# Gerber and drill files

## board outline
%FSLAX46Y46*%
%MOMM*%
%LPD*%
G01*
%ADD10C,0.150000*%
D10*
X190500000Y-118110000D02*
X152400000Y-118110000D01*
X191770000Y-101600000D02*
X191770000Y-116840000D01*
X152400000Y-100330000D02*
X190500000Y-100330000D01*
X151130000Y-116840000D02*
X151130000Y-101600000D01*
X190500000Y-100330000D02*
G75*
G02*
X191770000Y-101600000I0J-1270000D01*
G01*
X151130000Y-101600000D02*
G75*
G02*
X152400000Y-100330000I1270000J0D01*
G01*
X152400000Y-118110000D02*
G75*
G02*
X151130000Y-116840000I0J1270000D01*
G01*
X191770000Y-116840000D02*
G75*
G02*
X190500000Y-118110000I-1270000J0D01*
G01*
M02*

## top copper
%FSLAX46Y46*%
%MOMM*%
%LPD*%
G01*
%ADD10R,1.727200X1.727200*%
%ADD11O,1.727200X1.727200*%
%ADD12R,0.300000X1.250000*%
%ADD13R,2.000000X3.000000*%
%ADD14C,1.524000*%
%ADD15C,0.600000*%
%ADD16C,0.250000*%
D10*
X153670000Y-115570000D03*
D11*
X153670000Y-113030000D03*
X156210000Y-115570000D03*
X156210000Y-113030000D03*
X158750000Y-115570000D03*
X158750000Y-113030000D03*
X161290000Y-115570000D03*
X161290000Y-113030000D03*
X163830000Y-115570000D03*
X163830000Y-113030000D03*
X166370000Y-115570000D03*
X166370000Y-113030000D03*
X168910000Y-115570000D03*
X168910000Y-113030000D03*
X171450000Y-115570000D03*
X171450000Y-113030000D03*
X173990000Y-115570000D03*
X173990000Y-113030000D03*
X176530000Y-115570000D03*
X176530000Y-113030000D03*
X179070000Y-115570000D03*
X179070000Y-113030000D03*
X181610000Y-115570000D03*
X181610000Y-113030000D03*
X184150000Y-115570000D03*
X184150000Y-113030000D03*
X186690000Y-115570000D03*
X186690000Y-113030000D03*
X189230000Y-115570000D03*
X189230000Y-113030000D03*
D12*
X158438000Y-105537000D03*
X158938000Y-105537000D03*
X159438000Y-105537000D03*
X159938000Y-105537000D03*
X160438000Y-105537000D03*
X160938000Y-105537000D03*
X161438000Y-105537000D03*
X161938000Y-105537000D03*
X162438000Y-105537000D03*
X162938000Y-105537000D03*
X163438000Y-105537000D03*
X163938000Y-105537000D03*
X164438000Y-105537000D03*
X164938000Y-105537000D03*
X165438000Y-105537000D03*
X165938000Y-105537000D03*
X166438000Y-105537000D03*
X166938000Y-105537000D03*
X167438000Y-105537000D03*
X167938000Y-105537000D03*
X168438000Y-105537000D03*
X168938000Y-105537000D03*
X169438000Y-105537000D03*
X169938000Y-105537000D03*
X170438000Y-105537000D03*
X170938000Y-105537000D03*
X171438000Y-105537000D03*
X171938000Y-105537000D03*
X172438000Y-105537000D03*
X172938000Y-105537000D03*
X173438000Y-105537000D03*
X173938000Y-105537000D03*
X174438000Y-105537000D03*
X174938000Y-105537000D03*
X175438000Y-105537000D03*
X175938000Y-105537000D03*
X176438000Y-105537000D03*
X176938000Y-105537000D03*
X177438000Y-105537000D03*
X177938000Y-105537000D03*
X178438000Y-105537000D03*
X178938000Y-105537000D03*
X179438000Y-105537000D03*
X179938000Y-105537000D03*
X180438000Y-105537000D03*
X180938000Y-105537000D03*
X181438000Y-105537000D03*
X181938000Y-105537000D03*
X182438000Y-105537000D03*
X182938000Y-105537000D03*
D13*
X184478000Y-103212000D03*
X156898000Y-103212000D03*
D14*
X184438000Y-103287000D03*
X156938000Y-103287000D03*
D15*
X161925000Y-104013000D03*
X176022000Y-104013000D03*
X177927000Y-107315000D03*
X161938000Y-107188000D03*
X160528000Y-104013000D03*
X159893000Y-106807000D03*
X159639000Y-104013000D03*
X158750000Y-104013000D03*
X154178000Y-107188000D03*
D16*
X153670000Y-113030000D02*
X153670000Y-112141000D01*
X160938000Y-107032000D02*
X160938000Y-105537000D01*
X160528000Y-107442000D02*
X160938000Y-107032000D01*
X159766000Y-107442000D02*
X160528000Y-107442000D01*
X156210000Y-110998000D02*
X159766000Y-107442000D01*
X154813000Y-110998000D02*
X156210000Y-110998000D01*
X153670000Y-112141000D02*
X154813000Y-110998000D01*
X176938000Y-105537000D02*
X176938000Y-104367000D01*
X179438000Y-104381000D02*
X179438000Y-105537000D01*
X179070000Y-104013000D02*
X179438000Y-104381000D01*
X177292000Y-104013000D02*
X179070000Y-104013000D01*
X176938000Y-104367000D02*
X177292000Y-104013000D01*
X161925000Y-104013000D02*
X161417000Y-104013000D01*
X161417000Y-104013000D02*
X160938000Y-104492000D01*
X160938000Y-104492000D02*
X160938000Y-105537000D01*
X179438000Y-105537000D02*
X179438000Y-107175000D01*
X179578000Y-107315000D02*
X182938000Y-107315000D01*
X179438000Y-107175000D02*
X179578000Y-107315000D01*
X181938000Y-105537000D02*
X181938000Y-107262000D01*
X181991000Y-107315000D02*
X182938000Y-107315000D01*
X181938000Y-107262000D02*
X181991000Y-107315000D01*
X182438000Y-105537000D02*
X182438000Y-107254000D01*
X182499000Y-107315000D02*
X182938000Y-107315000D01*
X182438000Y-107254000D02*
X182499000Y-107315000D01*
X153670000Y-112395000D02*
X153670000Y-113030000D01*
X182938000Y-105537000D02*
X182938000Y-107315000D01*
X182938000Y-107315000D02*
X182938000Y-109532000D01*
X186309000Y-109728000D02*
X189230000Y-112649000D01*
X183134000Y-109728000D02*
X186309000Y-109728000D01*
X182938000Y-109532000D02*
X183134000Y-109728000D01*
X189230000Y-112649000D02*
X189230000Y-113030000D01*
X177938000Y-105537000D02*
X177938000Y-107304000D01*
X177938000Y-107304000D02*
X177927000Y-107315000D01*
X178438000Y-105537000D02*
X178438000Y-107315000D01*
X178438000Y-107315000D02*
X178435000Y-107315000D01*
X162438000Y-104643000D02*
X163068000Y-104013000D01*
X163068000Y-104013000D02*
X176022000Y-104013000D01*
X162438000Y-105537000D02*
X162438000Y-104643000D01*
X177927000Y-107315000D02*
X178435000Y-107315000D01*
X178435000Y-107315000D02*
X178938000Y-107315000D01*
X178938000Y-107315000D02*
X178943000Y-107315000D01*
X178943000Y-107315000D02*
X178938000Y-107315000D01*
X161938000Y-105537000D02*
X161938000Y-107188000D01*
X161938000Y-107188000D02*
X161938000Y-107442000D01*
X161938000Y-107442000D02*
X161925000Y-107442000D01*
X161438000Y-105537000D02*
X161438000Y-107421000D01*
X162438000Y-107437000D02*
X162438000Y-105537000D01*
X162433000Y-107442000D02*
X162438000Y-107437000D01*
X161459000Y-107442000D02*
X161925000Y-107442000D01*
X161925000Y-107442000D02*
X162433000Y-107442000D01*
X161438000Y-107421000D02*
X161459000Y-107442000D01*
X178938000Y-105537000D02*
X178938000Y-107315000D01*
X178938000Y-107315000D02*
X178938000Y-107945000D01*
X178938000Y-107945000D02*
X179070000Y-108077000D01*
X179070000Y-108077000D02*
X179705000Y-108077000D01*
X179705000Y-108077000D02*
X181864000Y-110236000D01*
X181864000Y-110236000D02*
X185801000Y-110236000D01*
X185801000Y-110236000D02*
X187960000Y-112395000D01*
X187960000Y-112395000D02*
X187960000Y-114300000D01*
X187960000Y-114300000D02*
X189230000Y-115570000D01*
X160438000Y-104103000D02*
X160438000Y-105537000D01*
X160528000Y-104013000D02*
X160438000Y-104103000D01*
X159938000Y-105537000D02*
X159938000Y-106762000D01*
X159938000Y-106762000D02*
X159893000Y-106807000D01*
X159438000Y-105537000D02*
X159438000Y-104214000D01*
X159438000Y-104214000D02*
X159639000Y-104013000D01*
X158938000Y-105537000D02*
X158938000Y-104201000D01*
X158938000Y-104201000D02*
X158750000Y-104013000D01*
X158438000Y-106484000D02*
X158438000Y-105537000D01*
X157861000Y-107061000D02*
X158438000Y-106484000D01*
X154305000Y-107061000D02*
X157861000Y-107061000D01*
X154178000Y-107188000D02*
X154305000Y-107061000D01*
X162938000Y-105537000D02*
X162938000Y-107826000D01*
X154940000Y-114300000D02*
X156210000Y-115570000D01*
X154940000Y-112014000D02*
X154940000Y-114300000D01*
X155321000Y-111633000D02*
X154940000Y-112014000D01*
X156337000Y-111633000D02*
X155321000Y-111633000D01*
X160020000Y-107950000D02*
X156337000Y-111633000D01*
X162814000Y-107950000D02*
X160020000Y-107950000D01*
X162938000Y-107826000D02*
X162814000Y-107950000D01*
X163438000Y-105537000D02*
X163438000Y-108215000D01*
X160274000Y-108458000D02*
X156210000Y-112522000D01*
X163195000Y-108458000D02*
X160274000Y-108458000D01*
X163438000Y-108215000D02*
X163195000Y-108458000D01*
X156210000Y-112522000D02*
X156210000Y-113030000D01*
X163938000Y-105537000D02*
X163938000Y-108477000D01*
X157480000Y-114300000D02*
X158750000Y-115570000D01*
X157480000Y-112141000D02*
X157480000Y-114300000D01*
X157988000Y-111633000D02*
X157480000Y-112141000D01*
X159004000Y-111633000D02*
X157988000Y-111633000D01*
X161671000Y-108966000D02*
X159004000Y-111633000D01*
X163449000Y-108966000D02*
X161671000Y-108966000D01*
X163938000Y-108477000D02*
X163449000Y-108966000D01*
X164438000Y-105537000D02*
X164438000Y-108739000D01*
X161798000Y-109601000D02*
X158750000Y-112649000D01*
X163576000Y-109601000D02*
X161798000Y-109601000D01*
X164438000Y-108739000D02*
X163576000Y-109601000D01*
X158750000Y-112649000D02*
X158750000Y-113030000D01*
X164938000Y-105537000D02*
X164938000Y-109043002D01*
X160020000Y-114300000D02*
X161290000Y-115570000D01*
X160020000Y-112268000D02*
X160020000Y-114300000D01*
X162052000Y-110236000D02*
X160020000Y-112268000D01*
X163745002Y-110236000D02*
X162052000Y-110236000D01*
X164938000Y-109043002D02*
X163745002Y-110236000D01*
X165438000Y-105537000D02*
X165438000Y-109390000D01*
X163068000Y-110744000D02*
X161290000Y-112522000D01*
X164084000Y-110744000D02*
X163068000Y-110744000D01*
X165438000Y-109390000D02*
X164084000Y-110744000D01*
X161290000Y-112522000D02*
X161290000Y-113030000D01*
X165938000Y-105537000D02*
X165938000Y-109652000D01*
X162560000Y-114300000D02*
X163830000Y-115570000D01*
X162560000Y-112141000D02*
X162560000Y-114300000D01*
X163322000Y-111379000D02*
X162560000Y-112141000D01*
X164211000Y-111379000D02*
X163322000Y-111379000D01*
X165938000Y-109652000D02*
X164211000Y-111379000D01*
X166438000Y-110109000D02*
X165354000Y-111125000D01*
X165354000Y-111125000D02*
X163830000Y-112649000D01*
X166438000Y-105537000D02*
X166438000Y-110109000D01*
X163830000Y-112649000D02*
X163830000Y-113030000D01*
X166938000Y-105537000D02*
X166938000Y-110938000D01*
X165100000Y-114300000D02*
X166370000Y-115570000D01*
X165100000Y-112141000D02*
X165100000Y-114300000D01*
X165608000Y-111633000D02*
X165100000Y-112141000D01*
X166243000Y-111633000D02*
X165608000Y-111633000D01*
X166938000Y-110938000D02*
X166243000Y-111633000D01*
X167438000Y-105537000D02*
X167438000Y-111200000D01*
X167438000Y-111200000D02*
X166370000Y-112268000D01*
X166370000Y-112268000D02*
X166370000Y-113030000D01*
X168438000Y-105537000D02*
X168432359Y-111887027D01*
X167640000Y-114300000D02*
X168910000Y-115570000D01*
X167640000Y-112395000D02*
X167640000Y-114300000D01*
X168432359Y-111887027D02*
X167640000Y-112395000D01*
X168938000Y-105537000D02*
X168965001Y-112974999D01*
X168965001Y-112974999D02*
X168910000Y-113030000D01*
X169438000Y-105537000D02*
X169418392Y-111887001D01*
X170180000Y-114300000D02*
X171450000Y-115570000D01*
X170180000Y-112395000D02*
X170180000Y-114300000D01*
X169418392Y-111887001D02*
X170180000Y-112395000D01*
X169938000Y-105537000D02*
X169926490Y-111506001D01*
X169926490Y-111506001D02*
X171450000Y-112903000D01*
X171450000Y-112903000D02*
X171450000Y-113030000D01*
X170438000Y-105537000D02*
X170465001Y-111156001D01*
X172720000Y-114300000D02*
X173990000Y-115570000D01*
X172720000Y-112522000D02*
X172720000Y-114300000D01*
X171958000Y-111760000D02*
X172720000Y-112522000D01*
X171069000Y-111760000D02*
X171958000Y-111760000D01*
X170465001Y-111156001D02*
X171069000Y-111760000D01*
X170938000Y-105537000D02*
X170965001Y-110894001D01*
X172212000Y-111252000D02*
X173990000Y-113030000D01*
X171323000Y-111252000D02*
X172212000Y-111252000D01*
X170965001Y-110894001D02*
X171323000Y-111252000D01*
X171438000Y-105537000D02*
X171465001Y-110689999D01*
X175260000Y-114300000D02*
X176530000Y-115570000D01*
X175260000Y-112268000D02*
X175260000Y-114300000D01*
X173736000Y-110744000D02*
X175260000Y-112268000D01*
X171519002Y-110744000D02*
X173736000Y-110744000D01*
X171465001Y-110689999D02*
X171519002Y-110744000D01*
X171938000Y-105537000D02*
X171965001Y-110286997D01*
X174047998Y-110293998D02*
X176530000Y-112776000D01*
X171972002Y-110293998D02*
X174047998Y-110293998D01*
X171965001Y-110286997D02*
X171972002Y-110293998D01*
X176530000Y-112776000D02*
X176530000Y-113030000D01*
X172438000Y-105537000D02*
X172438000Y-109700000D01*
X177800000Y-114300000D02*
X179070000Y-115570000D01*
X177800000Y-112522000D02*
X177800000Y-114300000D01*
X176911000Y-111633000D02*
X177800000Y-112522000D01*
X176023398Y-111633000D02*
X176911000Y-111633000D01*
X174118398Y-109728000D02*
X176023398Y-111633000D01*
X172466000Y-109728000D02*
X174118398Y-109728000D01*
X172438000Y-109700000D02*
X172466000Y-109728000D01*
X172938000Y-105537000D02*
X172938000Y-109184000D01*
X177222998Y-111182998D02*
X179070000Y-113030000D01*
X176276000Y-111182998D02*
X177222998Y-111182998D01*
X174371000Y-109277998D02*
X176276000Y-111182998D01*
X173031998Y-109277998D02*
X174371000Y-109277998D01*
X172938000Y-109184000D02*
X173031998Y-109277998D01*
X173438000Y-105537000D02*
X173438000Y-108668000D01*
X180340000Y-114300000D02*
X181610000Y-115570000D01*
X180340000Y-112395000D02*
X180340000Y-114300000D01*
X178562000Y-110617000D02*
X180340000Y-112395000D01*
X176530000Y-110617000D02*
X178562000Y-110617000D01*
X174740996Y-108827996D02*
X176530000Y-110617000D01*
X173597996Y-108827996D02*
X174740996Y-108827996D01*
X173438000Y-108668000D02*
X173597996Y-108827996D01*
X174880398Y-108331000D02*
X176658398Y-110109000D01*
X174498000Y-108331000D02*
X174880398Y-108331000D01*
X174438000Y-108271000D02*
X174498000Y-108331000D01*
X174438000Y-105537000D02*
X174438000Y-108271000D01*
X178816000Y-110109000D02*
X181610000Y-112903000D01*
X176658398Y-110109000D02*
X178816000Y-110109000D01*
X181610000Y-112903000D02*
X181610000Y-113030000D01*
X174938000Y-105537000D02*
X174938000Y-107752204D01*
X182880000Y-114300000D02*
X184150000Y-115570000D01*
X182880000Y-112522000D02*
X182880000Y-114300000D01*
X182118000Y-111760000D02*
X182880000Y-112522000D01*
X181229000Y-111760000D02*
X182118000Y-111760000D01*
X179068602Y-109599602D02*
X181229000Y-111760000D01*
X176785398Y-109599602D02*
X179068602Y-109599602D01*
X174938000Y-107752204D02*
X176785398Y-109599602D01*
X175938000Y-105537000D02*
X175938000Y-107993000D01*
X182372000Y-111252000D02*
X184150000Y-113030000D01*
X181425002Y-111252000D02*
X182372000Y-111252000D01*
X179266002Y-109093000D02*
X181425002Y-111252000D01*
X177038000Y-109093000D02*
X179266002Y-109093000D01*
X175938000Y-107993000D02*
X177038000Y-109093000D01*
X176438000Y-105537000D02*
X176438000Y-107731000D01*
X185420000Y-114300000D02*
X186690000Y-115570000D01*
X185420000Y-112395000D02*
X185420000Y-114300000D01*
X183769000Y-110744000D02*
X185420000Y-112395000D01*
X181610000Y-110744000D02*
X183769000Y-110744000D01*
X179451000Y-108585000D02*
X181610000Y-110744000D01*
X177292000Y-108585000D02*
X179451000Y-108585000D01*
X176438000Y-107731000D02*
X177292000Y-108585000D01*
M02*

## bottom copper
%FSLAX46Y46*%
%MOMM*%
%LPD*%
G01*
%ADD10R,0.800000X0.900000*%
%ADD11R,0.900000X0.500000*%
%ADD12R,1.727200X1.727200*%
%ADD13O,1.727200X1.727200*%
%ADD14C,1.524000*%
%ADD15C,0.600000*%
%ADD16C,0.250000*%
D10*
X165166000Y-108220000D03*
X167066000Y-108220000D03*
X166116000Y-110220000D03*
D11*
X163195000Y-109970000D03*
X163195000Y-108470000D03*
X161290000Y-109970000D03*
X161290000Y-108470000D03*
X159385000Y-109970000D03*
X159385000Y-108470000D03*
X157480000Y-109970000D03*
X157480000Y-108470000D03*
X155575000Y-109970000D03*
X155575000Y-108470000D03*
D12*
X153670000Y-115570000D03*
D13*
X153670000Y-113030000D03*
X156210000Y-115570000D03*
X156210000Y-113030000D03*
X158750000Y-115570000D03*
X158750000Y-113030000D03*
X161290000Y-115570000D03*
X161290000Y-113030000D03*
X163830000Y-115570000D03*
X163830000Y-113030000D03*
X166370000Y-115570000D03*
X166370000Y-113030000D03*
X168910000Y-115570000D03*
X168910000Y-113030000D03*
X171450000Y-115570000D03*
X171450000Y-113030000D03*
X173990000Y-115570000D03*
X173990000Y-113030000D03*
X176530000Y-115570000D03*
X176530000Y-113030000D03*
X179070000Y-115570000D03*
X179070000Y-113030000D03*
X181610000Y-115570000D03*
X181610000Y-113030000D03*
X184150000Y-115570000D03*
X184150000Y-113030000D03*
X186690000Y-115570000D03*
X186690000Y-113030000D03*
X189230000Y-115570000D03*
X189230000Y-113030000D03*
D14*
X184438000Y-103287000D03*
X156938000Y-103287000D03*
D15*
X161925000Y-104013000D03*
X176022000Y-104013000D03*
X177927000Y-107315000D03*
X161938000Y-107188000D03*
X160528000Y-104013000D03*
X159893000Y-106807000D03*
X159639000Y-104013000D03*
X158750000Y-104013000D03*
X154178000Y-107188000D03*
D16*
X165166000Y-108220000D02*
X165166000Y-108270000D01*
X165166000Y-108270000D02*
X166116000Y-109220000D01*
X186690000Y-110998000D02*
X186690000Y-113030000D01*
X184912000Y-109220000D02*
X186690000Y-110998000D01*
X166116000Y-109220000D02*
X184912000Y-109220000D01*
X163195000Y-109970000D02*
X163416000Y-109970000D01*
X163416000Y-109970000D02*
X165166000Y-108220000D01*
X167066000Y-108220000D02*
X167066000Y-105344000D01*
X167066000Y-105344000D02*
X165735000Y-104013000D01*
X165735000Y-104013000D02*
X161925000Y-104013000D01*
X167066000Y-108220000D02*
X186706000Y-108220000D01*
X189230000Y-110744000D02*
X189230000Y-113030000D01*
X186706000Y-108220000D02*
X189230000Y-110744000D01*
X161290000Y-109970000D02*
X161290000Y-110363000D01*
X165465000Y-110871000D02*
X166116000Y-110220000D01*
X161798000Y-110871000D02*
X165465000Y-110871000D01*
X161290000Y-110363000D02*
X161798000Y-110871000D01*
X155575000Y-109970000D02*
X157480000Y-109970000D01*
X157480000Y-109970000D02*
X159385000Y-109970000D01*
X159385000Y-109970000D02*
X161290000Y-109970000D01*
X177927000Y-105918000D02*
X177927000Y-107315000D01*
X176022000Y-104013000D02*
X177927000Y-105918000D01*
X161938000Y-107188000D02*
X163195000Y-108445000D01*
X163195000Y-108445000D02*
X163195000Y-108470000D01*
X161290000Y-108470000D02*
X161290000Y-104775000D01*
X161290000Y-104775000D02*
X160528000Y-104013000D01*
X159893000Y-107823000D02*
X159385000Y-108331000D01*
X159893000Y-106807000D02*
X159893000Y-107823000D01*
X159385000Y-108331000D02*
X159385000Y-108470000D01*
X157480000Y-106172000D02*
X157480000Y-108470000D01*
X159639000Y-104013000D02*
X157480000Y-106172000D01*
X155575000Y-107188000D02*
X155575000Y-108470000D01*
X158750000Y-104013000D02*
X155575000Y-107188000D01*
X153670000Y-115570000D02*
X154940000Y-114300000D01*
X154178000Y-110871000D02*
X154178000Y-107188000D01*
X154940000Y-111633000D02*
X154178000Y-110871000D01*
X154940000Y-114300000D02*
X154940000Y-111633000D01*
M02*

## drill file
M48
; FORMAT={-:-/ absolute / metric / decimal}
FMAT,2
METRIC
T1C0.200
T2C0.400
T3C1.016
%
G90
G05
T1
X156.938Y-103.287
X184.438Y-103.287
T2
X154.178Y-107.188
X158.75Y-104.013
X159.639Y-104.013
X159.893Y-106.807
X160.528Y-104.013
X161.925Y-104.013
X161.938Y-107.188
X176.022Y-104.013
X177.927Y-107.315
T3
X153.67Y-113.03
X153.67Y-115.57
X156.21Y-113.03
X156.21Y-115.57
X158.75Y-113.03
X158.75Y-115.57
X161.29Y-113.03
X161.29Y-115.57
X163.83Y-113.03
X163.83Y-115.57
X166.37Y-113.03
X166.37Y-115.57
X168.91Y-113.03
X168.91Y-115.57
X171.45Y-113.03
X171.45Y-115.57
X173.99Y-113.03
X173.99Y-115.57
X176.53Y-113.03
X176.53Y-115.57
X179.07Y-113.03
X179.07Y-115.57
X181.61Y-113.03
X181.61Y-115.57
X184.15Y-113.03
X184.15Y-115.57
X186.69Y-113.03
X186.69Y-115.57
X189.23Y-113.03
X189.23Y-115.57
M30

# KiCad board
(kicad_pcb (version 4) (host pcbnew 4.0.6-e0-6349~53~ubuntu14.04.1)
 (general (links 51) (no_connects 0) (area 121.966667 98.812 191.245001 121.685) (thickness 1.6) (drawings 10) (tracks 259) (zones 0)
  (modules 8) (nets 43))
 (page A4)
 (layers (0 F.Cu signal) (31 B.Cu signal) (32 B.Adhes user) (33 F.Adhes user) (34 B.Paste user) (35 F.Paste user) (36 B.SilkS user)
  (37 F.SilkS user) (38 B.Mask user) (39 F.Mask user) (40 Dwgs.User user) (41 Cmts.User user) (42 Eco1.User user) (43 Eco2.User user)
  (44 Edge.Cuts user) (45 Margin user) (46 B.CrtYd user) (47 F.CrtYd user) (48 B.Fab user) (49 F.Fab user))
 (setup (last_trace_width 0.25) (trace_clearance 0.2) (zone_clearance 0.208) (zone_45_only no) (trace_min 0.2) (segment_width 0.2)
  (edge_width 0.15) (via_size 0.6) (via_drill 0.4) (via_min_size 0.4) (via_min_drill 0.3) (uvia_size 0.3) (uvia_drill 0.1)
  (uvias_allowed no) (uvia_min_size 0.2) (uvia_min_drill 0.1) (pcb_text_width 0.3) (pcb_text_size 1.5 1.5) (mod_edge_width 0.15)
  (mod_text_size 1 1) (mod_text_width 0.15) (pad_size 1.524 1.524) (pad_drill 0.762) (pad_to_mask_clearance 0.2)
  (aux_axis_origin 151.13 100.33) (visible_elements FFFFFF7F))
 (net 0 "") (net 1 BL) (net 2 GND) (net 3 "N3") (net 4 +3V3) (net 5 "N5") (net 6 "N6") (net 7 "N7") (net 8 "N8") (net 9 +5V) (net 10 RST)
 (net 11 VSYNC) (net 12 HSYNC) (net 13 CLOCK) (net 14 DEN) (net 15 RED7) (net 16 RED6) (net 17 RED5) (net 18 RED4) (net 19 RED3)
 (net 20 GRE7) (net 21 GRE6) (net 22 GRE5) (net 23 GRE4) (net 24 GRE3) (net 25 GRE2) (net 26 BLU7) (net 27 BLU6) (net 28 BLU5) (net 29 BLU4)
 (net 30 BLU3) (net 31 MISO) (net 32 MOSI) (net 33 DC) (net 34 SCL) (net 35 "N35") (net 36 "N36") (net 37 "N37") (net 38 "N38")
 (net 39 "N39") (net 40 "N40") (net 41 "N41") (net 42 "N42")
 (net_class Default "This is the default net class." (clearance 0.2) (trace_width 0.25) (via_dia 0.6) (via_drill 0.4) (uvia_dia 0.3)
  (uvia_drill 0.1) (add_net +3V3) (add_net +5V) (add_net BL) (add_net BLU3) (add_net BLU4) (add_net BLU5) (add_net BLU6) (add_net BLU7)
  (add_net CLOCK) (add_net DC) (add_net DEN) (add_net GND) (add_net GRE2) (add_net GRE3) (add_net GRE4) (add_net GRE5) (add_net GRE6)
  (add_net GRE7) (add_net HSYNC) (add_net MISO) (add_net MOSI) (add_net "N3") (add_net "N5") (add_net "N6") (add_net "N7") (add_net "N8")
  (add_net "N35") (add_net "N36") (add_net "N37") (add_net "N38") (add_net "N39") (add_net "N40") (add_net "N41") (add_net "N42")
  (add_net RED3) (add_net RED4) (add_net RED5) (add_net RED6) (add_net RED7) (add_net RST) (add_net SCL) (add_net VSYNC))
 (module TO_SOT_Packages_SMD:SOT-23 (layer B.Cu) (at 166.116 109.22 270)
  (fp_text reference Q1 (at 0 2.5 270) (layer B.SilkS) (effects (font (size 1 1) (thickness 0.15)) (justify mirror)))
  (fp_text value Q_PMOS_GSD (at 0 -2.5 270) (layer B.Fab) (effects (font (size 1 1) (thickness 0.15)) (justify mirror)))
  (pad 1 smd rect (at -1 0.95 270) (size 0.9 0.8) (layers B.Cu B.Paste B.Mask) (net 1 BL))
  (pad 2 smd rect (at -1 -0.95 270) (size 0.9 0.8) (layers B.Cu B.Paste B.Mask) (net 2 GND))
  (pad 3 smd rect (at 1 0 270) (size 0.9 0.8) (layers B.Cu B.Paste B.Mask) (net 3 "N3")))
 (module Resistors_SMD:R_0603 (layer B.Cu) (at 163.195 109.22 90)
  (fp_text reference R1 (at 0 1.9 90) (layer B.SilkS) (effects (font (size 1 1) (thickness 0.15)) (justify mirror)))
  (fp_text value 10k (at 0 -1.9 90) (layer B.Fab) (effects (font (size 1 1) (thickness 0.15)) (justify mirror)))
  (pad 1 smd rect (at -0.75 0 90) (size 0.5 0.9) (layers B.Cu B.Paste B.Mask) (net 1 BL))
  (pad 2 smd rect (at 0.75 0 90) (size 0.5 0.9) (layers B.Cu B.Paste B.Mask) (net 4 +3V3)))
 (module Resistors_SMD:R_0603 (layer B.Cu) (at 161.29 109.22 90)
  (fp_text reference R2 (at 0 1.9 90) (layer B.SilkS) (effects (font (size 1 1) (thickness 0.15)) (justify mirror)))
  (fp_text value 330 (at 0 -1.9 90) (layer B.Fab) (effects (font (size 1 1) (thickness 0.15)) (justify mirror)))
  (pad 1 smd rect (at -0.75 0 90) (size 0.5 0.9) (layers B.Cu B.Paste B.Mask) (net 3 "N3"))
  (pad 2 smd rect (at 0.75 0 90) (size 0.5 0.9) (layers B.Cu B.Paste B.Mask) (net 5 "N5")))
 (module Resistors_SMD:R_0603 (layer B.Cu) (at 159.385 109.22 90)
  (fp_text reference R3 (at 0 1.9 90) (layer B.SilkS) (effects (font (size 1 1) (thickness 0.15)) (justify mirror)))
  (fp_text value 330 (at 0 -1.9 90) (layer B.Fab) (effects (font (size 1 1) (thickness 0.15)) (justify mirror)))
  (pad 1 smd rect (at -0.75 0 90) (size 0.5 0.9) (layers B.Cu B.Paste B.Mask) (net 3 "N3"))
  (pad 2 smd rect (at 0.75 0 90) (size 0.5 0.9) (layers B.Cu B.Paste B.Mask) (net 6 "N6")))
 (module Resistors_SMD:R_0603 (layer B.Cu) (at 157.48 109.22 90)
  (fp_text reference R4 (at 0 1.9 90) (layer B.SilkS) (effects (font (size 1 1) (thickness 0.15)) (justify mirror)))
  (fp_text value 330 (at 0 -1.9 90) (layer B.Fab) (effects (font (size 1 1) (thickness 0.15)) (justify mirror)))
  (pad 1 smd rect (at -0.75 0 90) (size 0.5 0.9) (layers B.Cu B.Paste B.Mask) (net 3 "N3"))
  (pad 2 smd rect (at 0.75 0 90) (size 0.5 0.9) (layers B.Cu B.Paste B.Mask) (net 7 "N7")))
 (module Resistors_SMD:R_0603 (layer B.Cu) (at 155.575 109.22 90)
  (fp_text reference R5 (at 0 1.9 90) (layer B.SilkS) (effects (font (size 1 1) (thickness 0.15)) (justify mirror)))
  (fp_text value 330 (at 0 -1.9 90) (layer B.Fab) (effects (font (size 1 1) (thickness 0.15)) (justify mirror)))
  (pad 1 smd rect (at -0.75 0 90) (size 0.5 0.9) (layers B.Cu B.Paste B.Mask) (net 3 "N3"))
  (pad 2 smd rect (at 0.75 0 90) (size 0.5 0.9) (layers B.Cu B.Paste B.Mask) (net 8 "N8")))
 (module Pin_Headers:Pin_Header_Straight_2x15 (layer F.Cu) (at 153.67 115.57 90)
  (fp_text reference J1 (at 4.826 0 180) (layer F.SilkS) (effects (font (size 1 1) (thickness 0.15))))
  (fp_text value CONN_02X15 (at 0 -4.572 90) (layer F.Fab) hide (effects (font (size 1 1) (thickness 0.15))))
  (pad 1 thru_hole rect (at 0 0 90) (size 1.7272 1.7272) (drill 1.016) (layers *.Cu *.Mask) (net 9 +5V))
  (pad 2 thru_hole oval (at 2.54 0 90) (size 1.7272 1.7272) (drill 1.016) (layers *.Cu *.Mask) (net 2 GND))
  (pad 3 thru_hole oval (at 0 2.54 90) (size 1.7272 1.7272) (drill 1.016) (layers *.Cu *.Mask) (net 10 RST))
  (pad 4 thru_hole oval (at 2.54 2.54 90) (size 1.7272 1.7272) (drill 1.016) (layers *.Cu *.Mask) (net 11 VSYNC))
  (pad 5 thru_hole oval (at 0 5.08 90) (size 1.7272 1.7272) (drill 1.016) (layers *.Cu *.Mask) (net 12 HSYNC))
  (pad 6 thru_hole oval (at 2.54 5.08 90) (size 1.7272 1.7272) (drill 1.016) (layers *.Cu *.Mask) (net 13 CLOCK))
  (pad 7 thru_hole oval (at 0 7.62 90) (size 1.7272 1.7272) (drill 1.016) (layers *.Cu *.Mask) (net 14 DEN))
  (pad 8 thru_hole oval (at 2.54 7.62 90) (size 1.7272 1.7272) (drill 1.016) (layers *.Cu *.Mask) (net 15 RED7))
  (pad 9 thru_hole oval (at 0 10.16 90) (size 1.7272 1.7272) (drill 1.016) (layers *.Cu *.Mask) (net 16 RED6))
  (pad 10 thru_hole oval (at 2.54 10.16 90) (size 1.7272 1.7272) (drill 1.016) (layers *.Cu *.Mask) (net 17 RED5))
  (pad 11 thru_hole oval (at 0 12.7 90) (size 1.7272 1.7272) (drill 1.016) (layers *.Cu *.Mask) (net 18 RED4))
  (pad 12 thru_hole oval (at 2.54 12.7 90) (size 1.7272 1.7272) (drill 1.016) (layers *.Cu *.Mask) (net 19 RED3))
  (pad 13 thru_hole oval (at 0 15.24 90) (size 1.7272 1.7272) (drill 1.016) (layers *.Cu *.Mask) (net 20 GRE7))
  (pad 14 thru_hole oval (at 2.54 15.24 90) (size 1.7272 1.7272) (drill 1.016) (layers *.Cu *.Mask) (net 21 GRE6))
  (pad 15 thru_hole oval (at 0 17.78 90) (size 1.7272 1.7272) (drill 1.016) (layers *.Cu *.Mask) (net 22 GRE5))
  (pad 16 thru_hole oval (at 2.54 17.78 90) (size 1.7272 1.7272) (drill 1.016) (layers *.Cu *.Mask) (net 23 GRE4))
  (pad 17 thru_hole oval (at 0 20.32 90) (size 1.7272 1.7272) (drill 1.016) (layers *.Cu *.Mask) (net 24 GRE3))
  (pad 18 thru_hole oval (at 2.54 20.32 90) (size 1.7272 1.7272) (drill 1.016) (layers *.Cu *.Mask) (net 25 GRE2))
  (pad 19 thru_hole oval (at 0 22.86 90) (size 1.7272 1.7272) (drill 1.016) (layers *.Cu *.Mask) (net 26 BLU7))
  (pad 20 thru_hole oval (at 2.54 22.86 90) (size 1.7272 1.7272) (drill 1.016) (layers *.Cu *.Mask) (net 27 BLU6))
  (pad 21 thru_hole oval (at 0 25.4 90) (size 1.7272 1.7272) (drill 1.016) (layers *.Cu *.Mask) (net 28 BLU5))
  (pad 22 thru_hole oval (at 2.54 25.4 90) (size 1.7272 1.7272) (drill 1.016) (layers *.Cu *.Mask) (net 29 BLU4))
  (pad 23 thru_hole oval (at 0 27.94 90) (size 1.7272 1.7272) (drill 1.016) (layers *.Cu *.Mask) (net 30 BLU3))
  (pad 24 thru_hole oval (at 2.54 27.94 90) (size 1.7272 1.7272) (drill 1.016) (layers *.Cu *.Mask) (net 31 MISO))
  (pad 25 thru_hole oval (at 0 30.48 90) (size 1.7272 1.7272) (drill 1.016) (layers *.Cu *.Mask) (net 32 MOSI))
  (pad 26 thru_hole oval (at 2.54 30.48 90) (size 1.7272 1.7272) (drill 1.016) (layers *.Cu *.Mask) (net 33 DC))
  (pad 27 thru_hole oval (at 0 33.02 90) (size 1.7272 1.7272) (drill 1.016) (layers *.Cu *.Mask) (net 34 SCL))
  (pad 28 thru_hole oval (at 2.54 33.02 90) (size 1.7272 1.7272) (drill 1.016) (layers *.Cu *.Mask) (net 1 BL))
  (pad 29 thru_hole oval (at 0 35.56 90) (size 1.7272 1.7272) (drill 1.016) (layers *.Cu *.Mask) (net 4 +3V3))
  (pad 30 thru_hole oval (at 2.54 35.56 90) (size 1.7272 1.7272) (drill 1.016) (layers *.Cu *.Mask) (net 2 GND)))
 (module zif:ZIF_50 (layer F.Cu) (at 170.688 105.537)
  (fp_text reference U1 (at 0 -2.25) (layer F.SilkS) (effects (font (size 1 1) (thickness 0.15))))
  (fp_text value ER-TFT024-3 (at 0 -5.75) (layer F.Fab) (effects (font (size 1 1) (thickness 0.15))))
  (pad 1 smd rect (at -12.25 0) (size 0.3 1.25) (layers F.Cu F.Paste F.Mask) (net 9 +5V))
  (pad 2 smd rect (at -11.75 0) (size 0.3 1.25) (layers F.Cu F.Paste F.Mask) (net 8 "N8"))
  (pad 3 smd rect (at -11.25 0) (size 0.3 1.25) (layers F.Cu F.Paste F.Mask) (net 7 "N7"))
  (pad 4 smd rect (at -10.75 0) (size 0.3 1.25) (layers F.Cu F.Paste F.Mask) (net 6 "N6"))
  (pad 5 smd rect (at -10.25 0) (size 0.3 1.25) (layers F.Cu F.Paste F.Mask) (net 5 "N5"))
  (pad 6 smd rect (at -9.75 0) (size 0.3 1.25) (layers F.Cu F.Paste F.Mask) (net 2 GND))
  (pad 7 smd rect (at -9.25 0) (size 0.3 1.25) (layers F.Cu F.Paste F.Mask) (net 4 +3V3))
  (pad 8 smd rect (at -8.75 0) (size 0.3 1.25) (layers F.Cu F.Paste F.Mask) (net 4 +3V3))
  (pad 9 smd rect (at -8.25 0) (size 0.3 1.25) (layers F.Cu F.Paste F.Mask) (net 4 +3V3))
  (pad 10 smd rect (at -7.75 0) (size 0.3 1.25) (layers F.Cu F.Paste F.Mask) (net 10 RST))
  (pad 11 smd rect (at -7.25 0) (size 0.3 1.25) (layers F.Cu F.Paste F.Mask) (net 11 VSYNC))
  (pad 12 smd rect (at -6.75 0) (size 0.3 1.25) (layers F.Cu F.Paste F.Mask) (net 12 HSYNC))
  (pad 13 smd rect (at -6.25 0) (size 0.3 1.25) (layers F.Cu F.Paste F.Mask) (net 13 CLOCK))
  (pad 14 smd rect (at -5.75 0) (size 0.3 1.25) (layers F.Cu F.Paste F.Mask) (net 14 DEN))
  (pad 15 smd rect (at -5.25 0) (size 0.3 1.25) (layers F.Cu F.Paste F.Mask) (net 15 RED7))
  (pad 16 smd rect (at -4.75 0) (size 0.3 1.25) (layers F.Cu F.Paste F.Mask) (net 16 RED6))
  (pad 17 smd rect (at -4.25 0) (size 0.3 1.25) (layers F.Cu F.Paste F.Mask) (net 17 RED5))
  (pad 18 smd rect (at -3.75 0) (size 0.3 1.25) (layers F.Cu F.Paste F.Mask) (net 18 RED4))
  (pad 19 smd rect (at -3.25 0) (size 0.3 1.25) (layers F.Cu F.Paste F.Mask) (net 19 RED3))
  (pad 20 smd rect (at -2.75 0) (size 0.3 1.25) (layers F.Cu F.Paste F.Mask) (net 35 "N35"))
  (pad 21 smd rect (at -2.25 0) (size 0.3 1.25) (layers F.Cu F.Paste F.Mask) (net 20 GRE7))
  (pad 22 smd rect (at -1.75 0) (size 0.3 1.25) (layers F.Cu F.Paste F.Mask) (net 21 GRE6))
  (pad 23 smd rect (at -1.25 0) (size 0.3 1.25) (layers F.Cu F.Paste F.Mask) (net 22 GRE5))
  (pad 24 smd rect (at -0.75 0) (size 0.3 1.25) (layers F.Cu F.Paste F.Mask) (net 23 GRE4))
  (pad 25 smd rect (at -0.25 0) (size 0.3 1.25) (layers F.Cu F.Paste F.Mask) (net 24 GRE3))
  (pad 26 smd rect (at 0.25 0) (size 0.3 1.25) (layers F.Cu F.Paste F.Mask) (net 25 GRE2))
  (pad 27 smd rect (at 0.75 0) (size 0.3 1.25) (layers F.Cu F.Paste F.Mask) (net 26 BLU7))
  (pad 28 smd rect (at 1.25 0) (size 0.3 1.25) (layers F.Cu F.Paste F.Mask) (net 27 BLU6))
  (pad 29 smd rect (at 1.75 0) (size 0.3 1.25) (layers F.Cu F.Paste F.Mask) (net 28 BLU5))
  (pad 30 smd rect (at 2.25 0) (size 0.3 1.25) (layers F.Cu F.Paste F.Mask) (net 29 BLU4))
  (pad 31 smd rect (at 2.75 0) (size 0.3 1.25) (layers F.Cu F.Paste F.Mask) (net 30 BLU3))
  (pad 32 smd rect (at 3.25 0) (size 0.3 1.25) (layers F.Cu F.Paste F.Mask) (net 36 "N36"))
  (pad 33 smd rect (at 3.75 0) (size 0.3 1.25) (layers F.Cu F.Paste F.Mask) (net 31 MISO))
  (pad 34 smd rect (at 4.25 0) (size 0.3 1.25) (layers F.Cu F.Paste F.Mask) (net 32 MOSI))
  (pad 35 smd rect (at 4.75 0) (size 0.3 1.25) (layers F.Cu F.Paste F.Mask) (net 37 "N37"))
  (pad 36 smd rect (at 5.25 0) (size 0.3 1.25) (layers F.Cu F.Paste F.Mask) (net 33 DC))
  (pad 37 smd rect (at 5.75 0) (size 0.3 1.25) (layers F.Cu F.Paste F.Mask) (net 34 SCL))
  (pad 38 smd rect (at 6.25 0) (size 0.3 1.25) (layers F.Cu F.Paste F.Mask) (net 2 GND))
  (pad 39 smd rect (at 6.75 0) (size 0.3 1.25) (layers F.Cu F.Paste F.Mask) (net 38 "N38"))
  (pad 40 smd rect (at 7.25 0) (size 0.3 1.25) (layers F.Cu F.Paste F.Mask) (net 4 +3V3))
  (pad 41 smd rect (at 7.75 0) (size 0.3 1.25) (layers F.Cu F.Paste F.Mask) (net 4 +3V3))
  (pad 42 smd rect (at 8.25 0) (size 0.3 1.25) (layers F.Cu F.Paste F.Mask) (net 4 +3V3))
  (pad 43 smd rect (at 8.75 0) (size 0.3 1.25) (layers F.Cu F.Paste F.Mask) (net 2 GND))
  (pad 44 smd rect (at 9.25 0) (size 0.3 1.25) (layers F.Cu F.Paste F.Mask) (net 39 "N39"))
  (pad 45 smd rect (at 9.75 0) (size 0.3 1.25) (layers F.Cu F.Paste F.Mask) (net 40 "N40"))
  (pad 46 smd rect (at 10.25 0) (size 0.3 1.25) (layers F.Cu F.Paste F.Mask) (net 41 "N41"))
  (pad 47 smd rect (at 10.75 0) (size 0.3 1.25) (layers F.Cu F.Paste F.Mask) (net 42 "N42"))
  (pad 48 smd rect (at 11.25 0) (size 0.3 1.25) (layers F.Cu F.Paste F.Mask) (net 2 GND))
  (pad 49 smd rect (at 11.75 0) (size 0.3 1.25) (layers F.Cu F.Paste F.Mask) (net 2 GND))
  (pad 50 smd rect (at 12.25 0) (size 0.3 1.25) (layers F.Cu F.Paste F.Mask) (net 2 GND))
  (pad G2 smd rect (at 13.79 -2.325) (size 2 3) (layers F.Cu F.Paste F.Mask))
  (pad G1 smd rect (at -13.79 -2.325) (size 2 3) (layers F.Cu F.Paste F.Mask))
  (pad G2 thru_hole circle (at 13.75 -2.25) (size 1.524 1.524) (drill 0.2) (layers *.Cu *.Mask))
  (pad G1 thru_hole circle (at -13.75 -2.25) (size 1.524 1.524) (drill 0.2) (layers *.Cu *.Mask)))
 (gr_line (start 190.5 118.11) (end 152.4 118.11) (angle 90) (layer Edge.Cuts) (width 0.15))
 (gr_line (start 191.77 101.6) (end 191.77 116.84) (angle 90) (layer Edge.Cuts) (width 0.15))
 (gr_line (start 152.4 100.33) (end 190.5 100.33) (angle 90) (layer Edge.Cuts) (width 0.15))
 (gr_line (start 151.13 116.84) (end 151.13 101.6) (angle 90) (layer Edge.Cuts) (width 0.15))
 (gr_arc (start 190.5 101.6) (end 190.5 100.33) (angle 90) (layer Edge.Cuts) (width 0.15))
 (gr_arc (start 152.4 101.6) (end 151.13 101.6) (angle 90) (layer Edge.Cuts) (width 0.15))
 (gr_arc (start 152.4 116.84) (end 152.4 118.11) (angle 90) (layer Edge.Cuts) (width 0.15))
 (gr_arc (start 190.5 116.84) (end 191.77 116.84) (angle 90) (layer Edge.Cuts) (width 0.15))
 (segment (start 165.166 108.22) (end 165.166 108.27) (width 0.25) (layer B.Cu) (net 1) (status C00000))
 (segment (start 165.166 108.27) (end 166.116 109.22) (width 0.25) (layer B.Cu) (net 1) (status 400000))
 (segment (start 186.69 110.998) (end 186.69 113.03) (width 0.25) (layer B.Cu) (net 1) (status 800000))
 (segment (start 184.912 109.22) (end 186.69 110.998) (width 0.25) (layer B.Cu) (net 1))
 (segment (start 166.116 109.22) (end 184.912 109.22) (width 0.25) (layer B.Cu) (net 1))
 (segment (start 163.195 109.97) (end 163.416 109.97) (width 0.25) (layer B.Cu) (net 1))
 (segment (start 163.416 109.97) (end 165.166 108.22) (width 0.25) (layer B.Cu) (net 1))
 (segment (start 153.67 113.03) (end 153.67 112.141) (width 0.25) (layer F.Cu) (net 2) (status 400000))
 (segment (start 160.938 107.032) (end 160.938 105.537) (width 0.25) (layer F.Cu) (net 2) (status 800000))
 (segment (start 160.528 107.442) (end 160.938 107.032) (width 0.25) (layer F.Cu) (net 2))
 (segment (start 159.766 107.442) (end 160.528 107.442) (width 0.25) (layer F.Cu) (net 2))
 (segment (start 156.21 110.998) (end 159.766 107.442) (width 0.25) (layer F.Cu) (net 2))
 (segment (start 154.813 110.998) (end 156.21 110.998) (width 0.25) (layer F.Cu) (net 2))
 (segment (start 153.67 112.141) (end 154.813 110.998) (width 0.25) (layer F.Cu) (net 2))
 (segment (start 176.938 105.537) (end 176.938 104.367) (width 0.25) (layer F.Cu) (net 2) (status 400000))
 (segment (start 179.438 104.381) (end 179.438 105.537) (width 0.25) (layer F.Cu) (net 2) (status 800000))
 (segment (start 179.07 104.013) (end 179.438 104.381) (width 0.25) (layer F.Cu) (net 2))
 (segment (start 177.292 104.013) (end 179.07 104.013) (width 0.25) (layer F.Cu) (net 2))
 (segment (start 176.938 104.367) (end 177.292 104.013) (width 0.25) (layer F.Cu) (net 2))
 (segment (start 167.066 108.22) (end 167.066 105.344) (width 0.25) (layer B.Cu) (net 2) (status 400000))
 (segment (start 167.066 105.344) (end 165.735 104.013) (width 0.25) (layer B.Cu) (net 2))
 (segment (start 165.735 104.013) (end 161.925 104.013) (width 0.25) (layer B.Cu) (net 2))
 (via (at 161.925 104.013) (size 0.6) (drill 0.4) (layers F.Cu B.Cu) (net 2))
 (segment (start 161.925 104.013) (end 161.417 104.013) (width 0.25) (layer F.Cu) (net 2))
 (segment (start 161.417 104.013) (end 160.938 104.492) (width 0.25) (layer F.Cu) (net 2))
 (segment (start 160.938 104.492) (end 160.938 105.537) (width 0.25) (layer F.Cu) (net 2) (status 800000))
 (segment (start 167.066 108.22) (end 186.706 108.22) (width 0.25) (layer B.Cu) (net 2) (status 400000))
 (segment (start 189.23 110.744) (end 189.23 113.03) (width 0.25) (layer B.Cu) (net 2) (status 800000))
 (segment (start 186.706 108.22) (end 189.23 110.744) (width 0.25) (layer B.Cu) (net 2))
 (segment (start 179.438 105.537) (end 179.438 107.175) (width 0.25) (layer F.Cu) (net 2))
 (segment (start 179.578 107.315) (end 182.938 107.315) (width 0.25) (layer F.Cu) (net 2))
 (segment (start 179.438 107.175) (end 179.578 107.315) (width 0.25) (layer F.Cu) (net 2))
 (segment (start 181.938 105.537) (end 181.938 107.262) (width 0.25) (layer F.Cu) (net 2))
 (segment (start 181.991 107.315) (end 182.938 107.315) (width 0.25) (layer F.Cu) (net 2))
 (segment (start 181.938 107.262) (end 181.991 107.315) (width 0.25) (layer F.Cu) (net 2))
 (segment (start 182.438 105.537) (end 182.438 107.254) (width 0.25) (layer F.Cu) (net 2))
 (segment (start 182.499 107.315) (end 182.938 107.315) (width 0.25) (layer F.Cu) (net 2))
 (segment (start 182.438 107.254) (end 182.499 107.315) (width 0.25) (layer F.Cu) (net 2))
 (segment (start 153.67 112.395) (end 153.67 113.03) (width 0.25) (layer F.Cu) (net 2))
 (segment (start 182.938 105.537) (end 182.938 107.315) (width 0.25) (layer F.Cu) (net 2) (status 10))
 (segment (start 182.938 107.315) (end 182.938 109.532) (width 0.25) (layer F.Cu) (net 2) (status 10))
 (segment (start 186.309 109.728) (end 189.23 112.649) (width 0.25) (layer F.Cu) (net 2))
 (segment (start 183.134 109.728) (end 186.309 109.728) (width 0.25) (layer F.Cu) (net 2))
 (segment (start 182.938 109.532) (end 183.134 109.728) (width 0.25) (layer F.Cu) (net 2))
 (segment (start 189.23 112.649) (end 189.23 113.03) (width 0.25) (layer F.Cu) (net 2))
 (segment (start 161.29 109.97) (end 161.29 110.363) (width 0.25) (layer B.Cu) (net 3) (status 400000))
 (segment (start 165.465 110.871) (end 166.116 110.22) (width 0.25) (layer B.Cu) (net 3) (status 800000))
 (segment (start 161.798 110.871) (end 165.465 110.871) (width 0.25) (layer B.Cu) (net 3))
 (segment (start 161.29 110.363) (end 161.798 110.871) (width 0.25) (layer B.Cu) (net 3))
 (segment (start 155.575 109.97) (end 157.48 109.97) (width 0.25) (layer B.Cu) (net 3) (status C00000))
 (segment (start 157.48 109.97) (end 159.385 109.97) (width 0.25) (layer B.Cu) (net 3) (status C00000))
 (segment (start 159.385 109.97) (end 161.29 109.97) (width 0.25) (layer B.Cu) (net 3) (status C00000))
 (segment (start 177.938 105.537) (end 177.938 107.304) (width 0.25) (layer F.Cu) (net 4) (status 400000))
 (segment (start 177.938 107.304) (end 177.927 107.315) (width 0.25) (layer F.Cu) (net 4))
 (segment (start 178.438 105.537) (end 178.438 107.315) (width 0.25) (layer F.Cu) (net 4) (status 400000))
 (segment (start 178.438 107.315) (end 178.435 107.315) (width 0.25) (layer F.Cu) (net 4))
 (via (at 176.022 104.013) (size 0.6) (drill 0.4) (layers F.Cu B.Cu) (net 4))
 (segment (start 162.438 104.643) (end 163.068 104.013) (width 0.25) (layer F.Cu) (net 4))
 (segment (start 163.068 104.013) (end 176.022 104.013) (width 0.25) (layer F.Cu) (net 4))
 (segment (start 162.438 105.537) (end 162.438 104.643) (width 0.25) (layer F.Cu) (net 4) (status 400000))
 (segment (start 177.927 107.315) (end 178.435 107.315) (width 0.25) (layer F.Cu) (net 4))
 (segment (start 178.435 107.315) (end 178.938 107.315) (width 0.25) (layer F.Cu) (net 4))
 (via (at 177.927 107.315) (size 0.6) (drill 0.4) (layers F.Cu B.Cu) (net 4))
 (segment (start 177.927 105.918) (end 177.927 107.315) (width 0.25) (layer B.Cu) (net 4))
 (segment (start 176.022 104.013) (end 177.927 105.918) (width 0.25) (layer B.Cu) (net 4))
 (segment (start 178.938 107.315) (end 178.943 107.315) (width 0.25) (layer F.Cu) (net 4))
 (segment (start 178.943 107.315) (end 178.938 107.315) (width 0.25) (layer F.Cu) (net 4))
 (via (at 161.938 107.188) (size 0.6) (drill 0.4) (layers F.Cu B.Cu) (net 4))
 (segment (start 161.938 107.188) (end 163.195 108.445) (width 0.25) (layer B.Cu) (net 4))
 (segment (start 163.195 108.445) (end 163.195 108.47) (width 0.25) (layer B.Cu) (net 4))
 (segment (start 161.938 105.537) (end 161.938 107.188) (width 0.25) (layer F.Cu) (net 4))
 (segment (start 161.938 107.188) (end 161.938 107.442) (width 0.25) (layer F.Cu) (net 4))
 (segment (start 161.938 107.442) (end 161.925 107.442) (width 0.25) (layer F.Cu) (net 4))
 (segment (start 161.438 105.537) (end 161.438 107.421) (width 0.25) (layer F.Cu) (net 4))
 (segment (start 162.438 107.437) (end 162.438 105.537) (width 0.25) (layer F.Cu) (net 4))
 (segment (start 162.433 107.442) (end 162.438 107.437) (width 0.25) (layer F.Cu) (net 4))
 (segment (start 161.459 107.442) (end 161.925 107.442) (width 0.25) (layer F.Cu) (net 4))
 (segment (start 161.925 107.442) (end 162.433 107.442) (width 0.25) (layer F.Cu) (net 4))
 (segment (start 161.438 107.421) (end 161.459 107.442) (width 0.25) (layer F.Cu) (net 4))
 (segment (start 178.938 105.537) (end 178.938 107.315) (width 0.25) (layer F.Cu) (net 4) (status 10))
 (segment (start 178.938 107.315) (end 178.938 107.945) (width 0.25) (layer F.Cu) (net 4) (status 10))
 (segment (start 178.938 107.945) (end 179.07 108.077) (width 0.25) (layer F.Cu) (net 4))
 (segment (start 179.07 108.077) (end 179.705 108.077) (width 0.25) (layer F.Cu) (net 4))
 (segment (start 179.705 108.077) (end 181.864 110.236) (width 0.25) (layer F.Cu) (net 4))
 (segment (start 181.864 110.236) (end 185.801 110.236) (width 0.25) (layer F.Cu) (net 4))
 (segment (start 185.801 110.236) (end 187.96 112.395) (width 0.25) (layer F.Cu) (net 4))
 (segment (start 187.96 112.395) (end 187.96 114.3) (width 0.25) (layer F.Cu) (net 4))
 (segment (start 187.96 114.3) (end 189.23 115.57) (width 0.25) (layer F.Cu) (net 4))
 (segment (start 161.29 108.47) (end 161.29 104.775) (width 0.25) (layer B.Cu) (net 5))
 (segment (start 160.438 104.103) (end 160.438 105.537) (width 0.25) (layer F.Cu) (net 5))
 (segment (start 160.528 104.013) (end 160.438 104.103) (width 0.25) (layer F.Cu) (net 5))
 (via (at 160.528 104.013) (size 0.6) (drill 0.4) (layers F.Cu B.Cu) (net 5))
 (segment (start 161.29 104.775) (end 160.528 104.013) (width 0.25) (layer B.Cu) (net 5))
 (segment (start 159.938 105.537) (end 159.938 106.762) (width 0.25) (layer F.Cu) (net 6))
 (segment (start 159.893 107.823) (end 159.385 108.331) (width 0.25) (layer B.Cu) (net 6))
 (segment (start 159.893 106.807) (end 159.893 107.823) (width 0.25) (layer B.Cu) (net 6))
 (via (at 159.893 106.807) (size 0.6) (drill 0.4) (layers F.Cu B.Cu) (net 6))
 (segment (start 159.938 106.762) (end 159.893 106.807) (width 0.25) (layer F.Cu) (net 6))
 (segment (start 159.385 108.331) (end 159.385 108.47) (width 0.25) (layer B.Cu) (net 6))
 (segment (start 159.438 105.537) (end 159.438 104.214) (width 0.25) (layer F.Cu) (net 7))
 (segment (start 157.48 106.172) (end 157.48 108.47) (width 0.25) (layer B.Cu) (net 7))
 (segment (start 159.639 104.013) (end 157.48 106.172) (width 0.25) (layer B.Cu) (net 7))
 (via (at 159.639 104.013) (size 0.6) (drill 0.4) (layers F.Cu B.Cu) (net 7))
 (segment (start 159.438 104.214) (end 159.639 104.013) (width 0.25) (layer F.Cu) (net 7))
 (segment (start 158.938 105.537) (end 158.938 104.201) (width 0.25) (layer F.Cu) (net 8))
 (segment (start 155.575 107.188) (end 155.575 108.47) (width 0.25) (layer B.Cu) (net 8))
 (segment (start 158.75 104.013) (end 155.575 107.188) (width 0.25) (layer B.Cu) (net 8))
 (via (at 158.75 104.013) (size 0.6) (drill 0.4) (layers F.Cu B.Cu) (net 8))
 (segment (start 158.938 104.201) (end 158.75 104.013) (width 0.25) (layer F.Cu) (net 8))
 (segment (start 153.67 115.57) (end 154.94 114.3) (width 0.25) (layer B.Cu) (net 9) (status 400000))
 (segment (start 158.438 106.484) (end 158.438 105.537) (width 0.25) (layer F.Cu) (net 9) (status 800000))
 (segment (start 157.861 107.061) (end 158.438 106.484) (width 0.25) (layer F.Cu) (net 9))
 (segment (start 154.305 107.061) (end 157.861 107.061) (width 0.25) (layer F.Cu) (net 9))
 (segment (start 154.178 107.188) (end 154.305 107.061) (width 0.25) (layer F.Cu) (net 9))
 (via (at 154.178 107.188) (size 0.6) (drill 0.4) (layers F.Cu B.Cu) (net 9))
 (segment (start 154.178 110.871) (end 154.178 107.188) (width 0.25) (layer B.Cu) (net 9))
 (segment (start 154.94 111.633) (end 154.178 110.871) (width 0.25) (layer B.Cu) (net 9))
 (segment (start 154.94 114.3) (end 154.94 111.633) (width 0.25) (layer B.Cu) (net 9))
 (segment (start 162.938 105.537) (end 162.938 107.826) (width 0.25) (layer F.Cu) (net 10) (status 10))
 (segment (start 154.94 114.3) (end 156.21 115.57) (width 0.25) (layer F.Cu) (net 10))
 (segment (start 154.94 112.014) (end 154.94 114.3) (width 0.25) (layer F.Cu) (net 10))
 (segment (start 155.321 111.633) (end 154.94 112.014) (width 0.25) (layer F.Cu) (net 10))
 (segment (start 156.337 111.633) (end 155.321 111.633) (width 0.25) (layer F.Cu) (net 10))
 (segment (start 160.02 107.95) (end 156.337 111.633) (width 0.25) (layer F.Cu) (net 10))
 (segment (start 162.814 107.95) (end 160.02 107.95) (width 0.25) (layer F.Cu) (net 10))
 (segment (start 162.938 107.826) (end 162.814 107.95) (width 0.25) (layer F.Cu) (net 10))
 (segment (start 163.438 105.537) (end 163.438 108.215) (width 0.25) (layer F.Cu) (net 11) (status 10))
 (segment (start 160.274 108.458) (end 156.21 112.522) (width 0.25) (layer F.Cu) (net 11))
 (segment (start 163.195 108.458) (end 160.274 108.458) (width 0.25) (layer F.Cu) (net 11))
 (segment (start 163.438 108.215) (end 163.195 108.458) (width 0.25) (layer F.Cu) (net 11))
 (segment (start 156.21 112.522) (end 156.21 113.03) (width 0.25) (layer F.Cu) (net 11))
 (segment (start 163.938 105.537) (end 163.938 108.477) (width 0.25) (layer F.Cu) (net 12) (status 10))
 (segment (start 157.48 114.3) (end 158.75 115.57) (width 0.25) (layer F.Cu) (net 12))
 (segment (start 157.48 112.141) (end 157.48 114.3) (width 0.25) (layer F.Cu) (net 12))
 (segment (start 157.988 111.633) (end 157.48 112.141) (width 0.25) (layer F.Cu) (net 12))
 (segment (start 159.004 111.633) (end 157.988 111.633) (width 0.25) (layer F.Cu) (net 12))
 (segment (start 161.671 108.966) (end 159.004 111.633) (width 0.25) (layer F.Cu) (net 12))
 (segment (start 163.449 108.966) (end 161.671 108.966) (width 0.25) (layer F.Cu) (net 12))
 (segment (start 163.938 108.477) (end 163.449 108.966) (width 0.25) (layer F.Cu) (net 12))
 (segment (start 164.438 105.537) (end 164.438 108.739) (width 0.25) (layer F.Cu) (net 13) (status 10))
 (segment (start 161.798 109.601) (end 158.75 112.649) (width 0.25) (layer F.Cu) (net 13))
 (segment (start 163.576 109.601) (end 161.798 109.601) (width 0.25) (layer F.Cu) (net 13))
 (segment (start 164.438 108.739) (end 163.576 109.601) (width 0.25) (layer F.Cu) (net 13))
 (segment (start 158.75 112.649) (end 158.75 113.03) (width 0.25) (layer F.Cu) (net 13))
 (segment (start 164.938 105.537) (end 164.938 109.043002) (width 0.25) (layer F.Cu) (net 14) (status 10))
 (segment (start 160.02 114.3) (end 161.29 115.57) (width 0.25) (layer F.Cu) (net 14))
 (segment (start 160.02 112.268) (end 160.02 114.3) (width 0.25) (layer F.Cu) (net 14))
 (segment (start 162.052 110.236) (end 160.02 112.268) (width 0.25) (layer F.Cu) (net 14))
 (segment (start 163.745002 110.236) (end 162.052 110.236) (width 0.25) (layer F.Cu) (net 14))
 (segment (start 164.938 109.043002) (end 163.745002 110.236) (width 0.25) (layer F.Cu) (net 14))
 (segment (start 165.438 105.537) (end 165.438 109.39) (width 0.25) (layer F.Cu) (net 15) (status 10))
 (segment (start 163.068 110.744) (end 161.29 112.522) (width 0.25) (layer F.Cu) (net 15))
 (segment (start 164.084 110.744) (end 163.068 110.744) (width 0.25) (layer F.Cu) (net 15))
 (segment (start 165.438 109.39) (end 164.084 110.744) (width 0.25) (layer F.Cu) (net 15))
 (segment (start 161.29 112.522) (end 161.29 113.03) (width 0.25) (layer F.Cu) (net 15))
 (segment (start 165.938 105.537) (end 165.938 109.652) (width 0.25) (layer F.Cu) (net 16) (status 10))
 (segment (start 162.56 114.3) (end 163.83 115.57) (width 0.25) (layer F.Cu) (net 16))
 (segment (start 162.56 112.141) (end 162.56 114.3) (width 0.25) (layer F.Cu) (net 16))
 (segment (start 163.322 111.379) (end 162.56 112.141) (width 0.25) (layer F.Cu) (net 16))
 (segment (start 164.211 111.379) (end 163.322 111.379) (width 0.25) (layer F.Cu) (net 16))
 (segment (start 165.938 109.652) (end 164.211 111.379) (width 0.25) (layer F.Cu) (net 16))
 (segment (start 166.438 110.109) (end 165.354 111.125) (width 0.25) (layer F.Cu) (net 17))
 (segment (start 165.354 111.125) (end 163.83 112.649) (width 0.25) (layer F.Cu) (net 17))
 (segment (start 166.438 105.537) (end 166.438 110.109) (width 0.25) (layer F.Cu) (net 17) (status 10))
 (segment (start 163.83 112.649) (end 163.83 113.03) (width 0.25) (layer F.Cu) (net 17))
 (segment (start 166.938 105.537) (end 166.938 110.938) (width 0.25) (layer F.Cu) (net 18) (status 10))
 (segment (start 165.1 114.3) (end 166.37 115.57) (width 0.25) (layer F.Cu) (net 18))
 (segment (start 165.1 112.141) (end 165.1 114.3) (width 0.25) (layer F.Cu) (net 18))
 (segment (start 165.608 111.633) (end 165.1 112.141) (width 0.25) (layer F.Cu) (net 18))
 (segment (start 166.243 111.633) (end 165.608 111.633) (width 0.25) (layer F.Cu) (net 18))
 (segment (start 166.938 110.938) (end 166.243 111.633) (width 0.25) (layer F.Cu) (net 18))
 (segment (start 167.438 105.537) (end 167.438 111.2) (width 0.25) (layer F.Cu) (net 19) (status 10))
 (segment (start 167.438 111.2) (end 166.37 112.268) (width 0.25) (layer F.Cu) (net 19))
 (segment (start 166.37 112.268) (end 166.37 113.03) (width 0.25) (layer F.Cu) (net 19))
 (segment (start 168.438 105.537) (end 168.432359 111.887027) (width 0.25) (layer F.Cu) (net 20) (status 10))
 (segment (start 167.64 114.3) (end 168.91 115.57) (width 0.25) (layer F.Cu) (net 20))
 (segment (start 167.64 112.395) (end 167.64 114.3) (width 0.25) (layer F.Cu) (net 20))
 (segment (start 168.432359 111.887027) (end 167.64 112.395) (width 0.25) (layer F.Cu) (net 20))
 (segment (start 168.938 105.537) (end 168.965001 112.974999) (width 0.25) (layer F.Cu) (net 21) (status 10))
 (segment (start 168.965001 112.974999) (end 168.91 113.03) (width 0.25) (layer F.Cu) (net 21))
 (segment (start 169.438 105.537) (end 169.418392 111.887001) (width 0.25) (layer F.Cu) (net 22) (status 10))
 (segment (start 170.18 114.3) (end 171.45 115.57) (width 0.25) (layer F.Cu) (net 22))
 (segment (start 170.18 112.395) (end 170.18 114.3) (width 0.25) (layer F.Cu) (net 22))
 (segment (start 169.418392 111.887001) (end 170.18 112.395) (width 0.25) (layer F.Cu) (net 22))
 (segment (start 169.938 105.537) (end 169.92649 111.506001) (width 0.25) (layer F.Cu) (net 23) (status 10))
 (segment (start 169.92649 111.506001) (end 171.45 112.903) (width 0.25) (layer F.Cu) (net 23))
 (segment (start 171.45 112.903) (end 171.45 113.03) (width 0.25) (layer F.Cu) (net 23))
 (segment (start 170.438 105.537) (end 170.465001 111.156001) (width 0.25) (layer F.Cu) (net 24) (status 10))
 (segment (start 172.72 114.3) (end 173.99 115.57) (width 0.25) (layer F.Cu) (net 24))
 (segment (start 172.72 112.522) (end 172.72 114.3) (width 0.25) (layer F.Cu) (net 24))
 (segment (start 171.958 111.76) (end 172.72 112.522) (width 0.25) (layer F.Cu) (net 24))
 (segment (start 171.069 111.76) (end 171.958 111.76) (width 0.25) (layer F.Cu) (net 24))
 (segment (start 170.465001 111.156001) (end 171.069 111.76) (width 0.25) (layer F.Cu) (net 24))
 (segment (start 170.938 105.537) (end 170.965001 110.894001) (width 0.25) (layer F.Cu) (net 25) (status 10))
 (segment (start 172.212 111.252) (end 173.99 113.03) (width 0.25) (layer F.Cu) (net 25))
 (segment (start 171.323 111.252) (end 172.212 111.252) (width 0.25) (layer F.Cu) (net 25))
 (segment (start 170.965001 110.894001) (end 171.323 111.252) (width 0.25) (layer F.Cu) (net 25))
 (segment (start 171.438 105.537) (end 171.465001 110.689999) (width 0.25) (layer F.Cu) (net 26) (status 10))
 (segment (start 175.26 114.3) (end 176.53 115.57) (width 0.25) (layer F.Cu) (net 26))
 (segment (start 175.26 112.268) (end 175.26 114.3) (width 0.25) (layer F.Cu) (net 26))
 (segment (start 173.736 110.744) (end 175.26 112.268) (width 0.25) (layer F.Cu) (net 26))
 (segment (start 171.519002 110.744) (end 173.736 110.744) (width 0.25) (layer F.Cu) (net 26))
 (segment (start 171.465001 110.689999) (end 171.519002 110.744) (width 0.25) (layer F.Cu) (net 26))
 (segment (start 171.938 105.537) (end 171.965001 110.286997) (width 0.25) (layer F.Cu) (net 27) (status 10))
 (segment (start 174.047998 110.293998) (end 176.53 112.776) (width 0.25) (layer F.Cu) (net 27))
 (segment (start 171.972002 110.293998) (end 174.047998 110.293998) (width 0.25) (layer F.Cu) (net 27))
 (segment (start 171.965001 110.286997) (end 171.972002 110.293998) (width 0.25) (layer F.Cu) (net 27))
 (segment (start 176.53 112.776) (end 176.53 113.03) (width 0.25) (layer F.Cu) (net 27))
 (segment (start 172.438 105.537) (end 172.438 109.7) (width 0.25) (layer F.Cu) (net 28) (status 10))
 (segment (start 177.8 114.3) (end 179.07 115.57) (width 0.25) (layer F.Cu) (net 28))
 (segment (start 177.8 112.522) (end 177.8 114.3) (width 0.25) (layer F.Cu) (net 28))
 (segment (start 176.911 111.633) (end 177.8 112.522) (width 0.25) (layer F.Cu) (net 28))
 (segment (start 176.023398 111.633) (end 176.911 111.633) (width 0.25) (layer F.Cu) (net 28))
 (segment (start 174.118398 109.728) (end 176.023398 111.633) (width 0.25) (layer F.Cu) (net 28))
 (segment (start 172.466 109.728) (end 174.118398 109.728) (width 0.25) (layer F.Cu) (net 28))
 (segment (start 172.438 109.7) (end 172.466 109.728) (width 0.25) (layer F.Cu) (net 28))
 (segment (start 172.938 105.537) (end 172.938 109.184) (width 0.25) (layer F.Cu) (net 29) (status 10))
 (segment (start 177.222998 111.182998) (end 179.07 113.03) (width 0.25) (layer F.Cu) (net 29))
 (segment (start 176.276 111.182998) (end 177.222998 111.182998) (width 0.25) (layer F.Cu) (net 29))
 (segment (start 174.371 109.277998) (end 176.276 111.182998) (width 0.25) (layer F.Cu) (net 29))
 (segment (start 173.031998 109.277998) (end 174.371 109.277998) (width 0.25) (layer F.Cu) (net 29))
 (segment (start 172.938 109.184) (end 173.031998 109.277998) (width 0.25) (layer F.Cu) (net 29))
 (segment (start 173.438 105.537) (end 173.438 108.668) (width 0.25) (layer F.Cu) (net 30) (status 10))
 (segment (start 180.34 114.3) (end 181.61 115.57) (width 0.25) (layer F.Cu) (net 30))
 (segment (start 180.34 112.395) (end 180.34 114.3) (width 0.25) (layer F.Cu) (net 30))
 (segment (start 178.562 110.617) (end 180.34 112.395) (width 0.25) (layer F.Cu) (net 30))
 (segment (start 176.53 110.617) (end 178.562 110.617) (width 0.25) (layer F.Cu) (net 30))
 (segment (start 174.740996 108.827996) (end 176.53 110.617) (width 0.25) (layer F.Cu) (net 30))
 (segment (start 173.597996 108.827996) (end 174.740996 108.827996) (width 0.25) (layer F.Cu) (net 30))
 (segment (start 173.438 108.668) (end 173.597996 108.827996) (width 0.25) (layer F.Cu) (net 30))
 (segment (start 174.880398 108.331) (end 176.658398 110.109) (width 0.25) (layer F.Cu) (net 31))
 (segment (start 174.498 108.331) (end 174.880398 108.331) (width 0.25) (layer F.Cu) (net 31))
 (segment (start 174.438 108.271) (end 174.498 108.331) (width 0.25) (layer F.Cu) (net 31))
 (segment (start 174.438 105.537) (end 174.438 108.271) (width 0.25) (layer F.Cu) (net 31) (status 10))
 (segment (start 178.816 110.109) (end 181.61 112.903) (width 0.25) (layer F.Cu) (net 31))
 (segment (start 176.658398 110.109) (end 178.816 110.109) (width 0.25) (layer F.Cu) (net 31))
 (segment (start 181.61 112.903) (end 181.61 113.03) (width 0.25) (layer F.Cu) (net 31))
 (segment (start 174.938 105.537) (end 174.938 107.752204) (width 0.25) (layer F.Cu) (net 32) (status 10))
 (segment (start 182.88 114.3) (end 184.15 115.57) (width 0.25) (layer F.Cu) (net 32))
 (segment (start 182.88 112.522) (end 182.88 114.3) (width 0.25) (layer F.Cu) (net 32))
 (segment (start 182.118 111.76) (end 182.88 112.522) (width 0.25) (layer F.Cu) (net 32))
 (segment (start 181.229 111.76) (end 182.118 111.76) (width 0.25) (layer F.Cu) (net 32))
 (segment (start 179.068602 109.599602) (end 181.229 111.76) (width 0.25) (layer F.Cu) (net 32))
 (segment (start 176.785398 109.599602) (end 179.068602 109.599602) (width 0.25) (layer F.Cu) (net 32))
 (segment (start 174.938 107.752204) (end 176.785398 109.599602) (width 0.25) (layer F.Cu) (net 32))
 (segment (start 175.938 105.537) (end 175.938 107.993) (width 0.25) (layer F.Cu) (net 33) (status 10))
 (segment (start 182.372 111.252) (end 184.15 113.03) (width 0.25) (layer F.Cu) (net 33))
 (segment (start 181.425002 111.252) (end 182.372 111.252) (width 0.25) (layer F.Cu) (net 33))
 (segment (start 179.266002 109.093) (end 181.425002 111.252) (width 0.25) (layer F.Cu) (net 33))
 (segment (start 177.038 109.093) (end 179.266002 109.093) (width 0.25) (layer F.Cu) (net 33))
 (segment (start 175.938 107.993) (end 177.038 109.093) (width 0.25) (layer F.Cu) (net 33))
 (segment (start 176.438 105.537) (end 176.438 107.731) (width 0.25) (layer F.Cu) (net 34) (status 10))
 (segment (start 185.42 114.3) (end 186.69 115.57) (width 0.25) (layer F.Cu) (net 34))
 (segment (start 185.42 112.395) (end 185.42 114.3) (width 0.25) (layer F.Cu) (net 34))
 (segment (start 183.769 110.744) (end 185.42 112.395) (width 0.25) (layer F.Cu) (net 34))
 (segment (start 181.61 110.744) (end 183.769 110.744) (width 0.25) (layer F.Cu) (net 34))
 (segment (start 179.451 108.585) (end 181.61 110.744) (width 0.25) (layer F.Cu) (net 34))
 (segment (start 177.292 108.585) (end 179.451 108.585) (width 0.25) (layer F.Cu) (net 34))
 (segment (start 176.438 107.731) (end 177.292 108.585) (width 0.25) (layer F.Cu) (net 34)))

